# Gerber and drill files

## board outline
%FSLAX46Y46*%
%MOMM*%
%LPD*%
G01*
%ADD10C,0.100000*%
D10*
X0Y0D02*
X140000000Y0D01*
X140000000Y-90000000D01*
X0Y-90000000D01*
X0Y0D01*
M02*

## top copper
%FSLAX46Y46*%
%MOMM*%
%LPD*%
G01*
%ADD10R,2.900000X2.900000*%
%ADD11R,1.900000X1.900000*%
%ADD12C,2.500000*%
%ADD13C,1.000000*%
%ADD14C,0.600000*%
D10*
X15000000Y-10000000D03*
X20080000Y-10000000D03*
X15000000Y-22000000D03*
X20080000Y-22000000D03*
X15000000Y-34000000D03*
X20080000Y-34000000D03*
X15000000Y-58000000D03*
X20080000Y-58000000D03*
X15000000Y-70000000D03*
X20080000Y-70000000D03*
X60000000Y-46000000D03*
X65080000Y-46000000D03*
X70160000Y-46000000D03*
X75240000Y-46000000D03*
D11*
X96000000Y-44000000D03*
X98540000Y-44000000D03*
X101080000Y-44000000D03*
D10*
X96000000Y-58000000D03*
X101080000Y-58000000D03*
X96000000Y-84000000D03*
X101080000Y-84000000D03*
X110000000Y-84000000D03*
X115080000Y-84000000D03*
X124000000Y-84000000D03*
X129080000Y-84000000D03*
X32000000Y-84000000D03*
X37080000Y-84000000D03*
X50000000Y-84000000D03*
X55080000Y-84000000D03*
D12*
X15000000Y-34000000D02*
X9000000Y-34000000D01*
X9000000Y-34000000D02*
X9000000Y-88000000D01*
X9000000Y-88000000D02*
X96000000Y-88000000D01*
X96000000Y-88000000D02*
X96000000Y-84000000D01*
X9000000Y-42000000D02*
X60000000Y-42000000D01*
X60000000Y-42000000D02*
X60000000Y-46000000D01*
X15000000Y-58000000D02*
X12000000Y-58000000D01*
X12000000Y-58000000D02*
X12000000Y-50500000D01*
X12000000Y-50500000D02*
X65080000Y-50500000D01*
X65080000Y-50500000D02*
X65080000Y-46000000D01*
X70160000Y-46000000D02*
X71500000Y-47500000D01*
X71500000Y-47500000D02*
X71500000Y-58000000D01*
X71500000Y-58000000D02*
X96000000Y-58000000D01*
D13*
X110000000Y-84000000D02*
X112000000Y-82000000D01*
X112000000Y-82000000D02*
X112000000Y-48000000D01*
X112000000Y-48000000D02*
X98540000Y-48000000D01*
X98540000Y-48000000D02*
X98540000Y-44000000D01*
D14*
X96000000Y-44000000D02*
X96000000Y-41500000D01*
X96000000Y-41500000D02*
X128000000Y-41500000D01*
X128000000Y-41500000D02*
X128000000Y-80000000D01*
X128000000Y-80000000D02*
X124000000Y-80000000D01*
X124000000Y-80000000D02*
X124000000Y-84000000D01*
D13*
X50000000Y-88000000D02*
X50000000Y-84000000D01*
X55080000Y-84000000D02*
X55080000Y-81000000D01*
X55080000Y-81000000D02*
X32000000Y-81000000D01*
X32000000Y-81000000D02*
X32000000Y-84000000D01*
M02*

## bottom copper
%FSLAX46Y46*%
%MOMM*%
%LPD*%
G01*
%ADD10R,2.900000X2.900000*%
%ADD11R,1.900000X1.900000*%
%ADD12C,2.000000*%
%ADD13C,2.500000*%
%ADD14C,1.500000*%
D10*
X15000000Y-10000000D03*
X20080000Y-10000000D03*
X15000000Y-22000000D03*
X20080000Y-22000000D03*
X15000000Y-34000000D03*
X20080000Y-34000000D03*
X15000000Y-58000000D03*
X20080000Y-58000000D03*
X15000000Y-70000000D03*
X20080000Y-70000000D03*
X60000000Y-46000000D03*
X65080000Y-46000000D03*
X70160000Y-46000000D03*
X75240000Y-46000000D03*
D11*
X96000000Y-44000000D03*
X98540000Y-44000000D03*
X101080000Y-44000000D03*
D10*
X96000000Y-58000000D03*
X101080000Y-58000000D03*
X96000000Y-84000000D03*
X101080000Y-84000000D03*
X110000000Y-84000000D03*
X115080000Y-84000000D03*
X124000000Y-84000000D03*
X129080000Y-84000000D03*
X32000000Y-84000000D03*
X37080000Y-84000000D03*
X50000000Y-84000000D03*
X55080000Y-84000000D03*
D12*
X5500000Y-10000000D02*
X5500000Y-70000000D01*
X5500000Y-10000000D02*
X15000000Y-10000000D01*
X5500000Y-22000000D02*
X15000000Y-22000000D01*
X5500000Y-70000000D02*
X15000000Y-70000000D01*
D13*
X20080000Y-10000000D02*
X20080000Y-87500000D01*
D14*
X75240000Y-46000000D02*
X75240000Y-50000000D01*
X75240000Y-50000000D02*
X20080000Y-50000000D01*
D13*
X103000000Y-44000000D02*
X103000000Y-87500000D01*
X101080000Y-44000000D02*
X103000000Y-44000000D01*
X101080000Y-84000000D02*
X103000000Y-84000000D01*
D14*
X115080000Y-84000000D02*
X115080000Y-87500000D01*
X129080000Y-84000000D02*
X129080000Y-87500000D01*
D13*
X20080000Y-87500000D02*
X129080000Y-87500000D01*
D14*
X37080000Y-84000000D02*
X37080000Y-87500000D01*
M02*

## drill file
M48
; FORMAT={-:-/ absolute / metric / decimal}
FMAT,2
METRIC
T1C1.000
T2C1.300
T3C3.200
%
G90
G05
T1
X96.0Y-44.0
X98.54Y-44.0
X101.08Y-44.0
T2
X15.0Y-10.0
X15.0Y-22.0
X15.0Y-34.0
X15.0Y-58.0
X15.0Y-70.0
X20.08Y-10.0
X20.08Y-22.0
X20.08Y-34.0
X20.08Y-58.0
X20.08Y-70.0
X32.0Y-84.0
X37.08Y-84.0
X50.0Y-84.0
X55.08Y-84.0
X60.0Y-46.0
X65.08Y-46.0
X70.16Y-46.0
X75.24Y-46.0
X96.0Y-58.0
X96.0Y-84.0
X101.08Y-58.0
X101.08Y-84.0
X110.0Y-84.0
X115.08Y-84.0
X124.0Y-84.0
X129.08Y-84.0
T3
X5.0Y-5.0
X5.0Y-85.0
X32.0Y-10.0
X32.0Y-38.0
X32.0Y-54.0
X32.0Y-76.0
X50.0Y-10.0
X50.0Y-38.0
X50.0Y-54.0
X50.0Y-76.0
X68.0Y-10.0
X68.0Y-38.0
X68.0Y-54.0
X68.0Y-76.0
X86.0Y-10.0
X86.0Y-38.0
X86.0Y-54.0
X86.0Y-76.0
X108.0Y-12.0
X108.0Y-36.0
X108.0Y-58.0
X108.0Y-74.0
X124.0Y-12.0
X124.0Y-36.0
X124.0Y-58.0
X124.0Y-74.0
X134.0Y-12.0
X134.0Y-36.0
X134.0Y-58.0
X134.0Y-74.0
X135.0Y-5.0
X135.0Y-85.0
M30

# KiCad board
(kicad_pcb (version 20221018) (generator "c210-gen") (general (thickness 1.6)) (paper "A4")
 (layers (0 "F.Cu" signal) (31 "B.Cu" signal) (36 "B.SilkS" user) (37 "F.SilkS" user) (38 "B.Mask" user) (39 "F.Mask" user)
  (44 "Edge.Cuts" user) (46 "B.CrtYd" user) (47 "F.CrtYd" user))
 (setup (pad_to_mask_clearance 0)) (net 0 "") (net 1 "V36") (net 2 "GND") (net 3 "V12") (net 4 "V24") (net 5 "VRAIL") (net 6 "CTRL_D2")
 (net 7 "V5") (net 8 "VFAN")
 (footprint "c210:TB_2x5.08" (layer "F.Cu") (at 15 10)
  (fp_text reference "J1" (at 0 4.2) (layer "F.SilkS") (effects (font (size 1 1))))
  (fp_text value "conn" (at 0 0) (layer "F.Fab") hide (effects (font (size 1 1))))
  (pad "1" thru_hole rect (at 0.0 0) (size 2.9 2.9) (drill 1.3) (layers "*.Cu" "*.Mask") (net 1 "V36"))
  (pad "2" thru_hole rect (at 5.08 0) (size 2.9 2.9) (drill 1.3) (layers "*.Cu" "*.Mask") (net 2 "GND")))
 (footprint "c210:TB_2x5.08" (layer "F.Cu") (at 15 22)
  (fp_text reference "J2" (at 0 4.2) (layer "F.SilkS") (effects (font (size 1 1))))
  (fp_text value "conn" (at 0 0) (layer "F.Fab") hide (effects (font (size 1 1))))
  (pad "1" thru_hole rect (at 0.0 0) (size 2.9 2.9) (drill 1.3) (layers "*.Cu" "*.Mask") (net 1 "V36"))
  (pad "2" thru_hole rect (at 5.08 0) (size 2.9 2.9) (drill 1.3) (layers "*.Cu" "*.Mask") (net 2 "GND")))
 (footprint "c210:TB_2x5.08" (layer "F.Cu") (at 15 34)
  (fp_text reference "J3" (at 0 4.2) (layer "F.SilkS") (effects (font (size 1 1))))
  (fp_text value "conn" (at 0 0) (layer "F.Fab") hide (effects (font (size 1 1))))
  (pad "1" thru_hole rect (at 0.0 0) (size 2.9 2.9) (drill 1.3) (layers "*.Cu" "*.Mask") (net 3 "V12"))
  (pad "2" thru_hole rect (at 5.08 0) (size 2.9 2.9) (drill 1.3) (layers "*.Cu" "*.Mask") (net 2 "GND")))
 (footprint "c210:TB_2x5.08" (layer "F.Cu") (at 15 58)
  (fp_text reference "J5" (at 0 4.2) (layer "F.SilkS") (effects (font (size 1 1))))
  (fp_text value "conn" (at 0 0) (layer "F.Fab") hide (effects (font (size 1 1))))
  (pad "1" thru_hole rect (at 0.0 0) (size 2.9 2.9) (drill 1.3) (layers "*.Cu" "*.Mask") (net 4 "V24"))
  (pad "2" thru_hole rect (at 5.08 0) (size 2.9 2.9) (drill 1.3) (layers "*.Cu" "*.Mask") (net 2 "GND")))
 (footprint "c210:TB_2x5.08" (layer "F.Cu") (at 15 70)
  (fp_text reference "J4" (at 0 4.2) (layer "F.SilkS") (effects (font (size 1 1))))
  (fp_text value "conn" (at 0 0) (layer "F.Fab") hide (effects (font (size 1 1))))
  (pad "1" thru_hole rect (at 0.0 0) (size 2.9 2.9) (drill 1.3) (layers "*.Cu" "*.Mask") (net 1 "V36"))
  (pad "2" thru_hole rect (at 5.08 0) (size 2.9 2.9) (drill 1.3) (layers "*.Cu" "*.Mask") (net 2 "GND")))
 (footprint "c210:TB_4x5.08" (layer "F.Cu") (at 60 46)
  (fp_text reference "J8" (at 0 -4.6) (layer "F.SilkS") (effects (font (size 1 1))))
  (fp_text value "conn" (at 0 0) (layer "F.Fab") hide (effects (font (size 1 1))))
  (pad "1" thru_hole rect (at 0.0 0) (size 2.9 2.9) (drill 1.3) (layers "*.Cu" "*.Mask") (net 3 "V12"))
  (pad "2" thru_hole rect (at 5.08 0) (size 2.9 2.9) (drill 1.3) (layers "*.Cu" "*.Mask") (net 4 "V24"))
  (pad "3" thru_hole rect (at 10.16 0) (size 2.9 2.9) (drill 1.3) (layers "*.Cu" "*.Mask") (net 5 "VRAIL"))
  (pad "4" thru_hole rect (at 15.24 0) (size 2.9 2.9) (drill 1.3) (layers "*.Cu" "*.Mask") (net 2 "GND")))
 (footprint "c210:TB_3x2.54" (layer "F.Cu") (at 96 44)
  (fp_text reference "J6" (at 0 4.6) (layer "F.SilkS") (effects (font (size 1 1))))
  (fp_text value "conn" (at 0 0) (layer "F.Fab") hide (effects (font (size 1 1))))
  (pad "1" thru_hole rect (at 0.0 0) (size 1.9 1.9) (drill 1.0) (layers "*.Cu" "*.Mask") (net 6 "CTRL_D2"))
  (pad "2" thru_hole rect (at 2.54 0) (size 1.9 1.9) (drill 1.0) (layers "*.Cu" "*.Mask") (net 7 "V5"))
  (pad "3" thru_hole rect (at 5.08 0) (size 1.9 1.9) (drill 1.0) (layers "*.Cu" "*.Mask") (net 2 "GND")))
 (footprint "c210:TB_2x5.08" (layer "F.Cu") (at 96 58)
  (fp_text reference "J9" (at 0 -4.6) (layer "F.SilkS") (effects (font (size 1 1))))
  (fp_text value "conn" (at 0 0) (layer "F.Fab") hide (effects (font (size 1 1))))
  (pad "1" thru_hole rect (at 0.0 0) (size 2.9 2.9) (drill 1.3) (layers "*.Cu" "*.Mask") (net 5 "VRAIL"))
  (pad "2" thru_hole rect (at 5.08 0) (size 2.9 2.9) (drill 1.3) (layers "*.Cu" "*.Mask") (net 2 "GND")))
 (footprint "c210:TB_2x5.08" (layer "F.Cu") (at 96 84)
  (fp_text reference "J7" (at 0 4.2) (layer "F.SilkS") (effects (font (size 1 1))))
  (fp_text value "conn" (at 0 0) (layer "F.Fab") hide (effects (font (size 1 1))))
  (pad "1" thru_hole rect (at 0.0 0) (size 2.9 2.9) (drill 1.3) (layers "*.Cu" "*.Mask") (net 3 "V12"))
  (pad "2" thru_hole rect (at 5.08 0) (size 2.9 2.9) (drill 1.3) (layers "*.Cu" "*.Mask") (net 2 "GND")))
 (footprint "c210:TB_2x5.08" (layer "F.Cu") (at 110 84)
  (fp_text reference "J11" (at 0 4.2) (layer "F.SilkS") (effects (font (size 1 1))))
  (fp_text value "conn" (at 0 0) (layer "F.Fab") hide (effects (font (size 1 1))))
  (pad "1" thru_hole rect (at 0.0 0) (size 2.9 2.9) (drill 1.3) (layers "*.Cu" "*.Mask") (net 7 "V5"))
  (pad "2" thru_hole rect (at 5.08 0) (size 2.9 2.9) (drill 1.3) (layers "*.Cu" "*.Mask") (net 2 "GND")))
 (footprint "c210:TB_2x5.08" (layer "F.Cu") (at 124 84)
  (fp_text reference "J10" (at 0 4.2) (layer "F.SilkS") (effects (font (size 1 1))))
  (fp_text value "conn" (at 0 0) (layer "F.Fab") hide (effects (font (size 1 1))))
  (pad "1" thru_hole rect (at 0.0 0) (size 2.9 2.9) (drill 1.3) (layers "*.Cu" "*.Mask") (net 6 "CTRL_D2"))
  (pad "2" thru_hole rect (at 5.08 0) (size 2.9 2.9) (drill 1.3) (layers "*.Cu" "*.Mask") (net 2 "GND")))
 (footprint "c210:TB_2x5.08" (layer "F.Cu") (at 32 84)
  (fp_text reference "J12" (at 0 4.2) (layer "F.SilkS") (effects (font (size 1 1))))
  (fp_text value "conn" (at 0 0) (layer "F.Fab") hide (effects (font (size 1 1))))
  (pad "1" thru_hole rect (at 0.0 0) (size 2.9 2.9) (drill 1.3) (layers "*.Cu" "*.Mask") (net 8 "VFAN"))
  (pad "2" thru_hole rect (at 5.08 0) (size 2.9 2.9) (drill 1.3) (layers "*.Cu" "*.Mask") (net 2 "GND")))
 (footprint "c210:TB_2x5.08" (layer "F.Cu") (at 50 84)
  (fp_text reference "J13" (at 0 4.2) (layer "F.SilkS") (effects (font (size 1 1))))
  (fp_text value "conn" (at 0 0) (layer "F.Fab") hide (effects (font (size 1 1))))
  (pad "1" thru_hole rect (at 0.0 0) (size 2.9 2.9) (drill 1.3) (layers "*.Cu" "*.Mask") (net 3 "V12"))
  (pad "2" thru_hole rect (at 5.08 0) (size 2.9 2.9) (drill 1.3) (layers "*.Cu" "*.Mask") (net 8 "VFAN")))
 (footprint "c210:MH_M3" (layer "F.Cu") (at 5 5)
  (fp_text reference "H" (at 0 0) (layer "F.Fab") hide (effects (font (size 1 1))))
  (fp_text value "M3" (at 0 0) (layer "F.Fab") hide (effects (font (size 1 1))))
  (pad "" np_thru_hole circle (at 0 0) (size 3.2 3.2) (drill 3.2) (layers "F.Mask" "B.Mask")))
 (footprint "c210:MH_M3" (layer "F.Cu") (at 135 5)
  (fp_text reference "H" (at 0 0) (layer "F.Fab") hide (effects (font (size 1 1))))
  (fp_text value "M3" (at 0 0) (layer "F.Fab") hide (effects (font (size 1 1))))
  (pad "" np_thru_hole circle (at 0 0) (size 3.2 3.2) (drill 3.2) (layers "F.Mask" "B.Mask")))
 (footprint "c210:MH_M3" (layer "F.Cu") (at 5 85)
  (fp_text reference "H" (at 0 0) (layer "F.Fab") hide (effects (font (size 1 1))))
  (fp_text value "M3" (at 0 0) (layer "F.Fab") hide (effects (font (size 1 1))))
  (pad "" np_thru_hole circle (at 0 0) (size 3.2 3.2) (drill 3.2) (layers "F.Mask" "B.Mask")))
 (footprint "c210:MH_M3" (layer "F.Cu") (at 135 85)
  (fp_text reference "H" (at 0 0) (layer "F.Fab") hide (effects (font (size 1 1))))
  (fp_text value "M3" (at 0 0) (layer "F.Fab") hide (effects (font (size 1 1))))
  (pad "" np_thru_hole circle (at 0 0) (size 3.2 3.2) (drill 3.2) (layers "F.Mask" "B.Mask")))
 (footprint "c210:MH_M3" (layer "F.Cu") (at 32 10)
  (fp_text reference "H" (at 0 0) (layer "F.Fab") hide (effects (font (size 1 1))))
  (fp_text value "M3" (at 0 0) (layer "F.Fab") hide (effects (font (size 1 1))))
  (pad "" np_thru_hole circle (at 0 0) (size 3.2 3.2) (drill 3.2) (layers "F.Mask" "B.Mask")))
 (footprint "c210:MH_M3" (layer "F.Cu") (at 32 38)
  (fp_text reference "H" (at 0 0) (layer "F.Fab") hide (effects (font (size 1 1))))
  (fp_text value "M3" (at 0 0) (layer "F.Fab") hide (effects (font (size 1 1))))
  (pad "" np_thru_hole circle (at 0 0) (size 3.2 3.2) (drill 3.2) (layers "F.Mask" "B.Mask")))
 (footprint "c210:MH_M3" (layer "F.Cu") (at 32 54)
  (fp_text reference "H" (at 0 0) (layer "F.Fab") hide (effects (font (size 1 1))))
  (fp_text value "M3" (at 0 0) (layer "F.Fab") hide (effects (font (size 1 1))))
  (pad "" np_thru_hole circle (at 0 0) (size 3.2 3.2) (drill 3.2) (layers "F.Mask" "B.Mask")))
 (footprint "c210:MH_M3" (layer "F.Cu") (at 32 76)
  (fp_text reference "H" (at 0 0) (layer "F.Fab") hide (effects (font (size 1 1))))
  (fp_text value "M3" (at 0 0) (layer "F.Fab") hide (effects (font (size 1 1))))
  (pad "" np_thru_hole circle (at 0 0) (size 3.2 3.2) (drill 3.2) (layers "F.Mask" "B.Mask")))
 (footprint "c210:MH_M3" (layer "F.Cu") (at 50 10)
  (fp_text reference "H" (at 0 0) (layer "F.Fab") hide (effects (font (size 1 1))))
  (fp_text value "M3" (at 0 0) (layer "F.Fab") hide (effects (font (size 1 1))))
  (pad "" np_thru_hole circle (at 0 0) (size 3.2 3.2) (drill 3.2) (layers "F.Mask" "B.Mask")))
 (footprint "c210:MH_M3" (layer "F.Cu") (at 50 38)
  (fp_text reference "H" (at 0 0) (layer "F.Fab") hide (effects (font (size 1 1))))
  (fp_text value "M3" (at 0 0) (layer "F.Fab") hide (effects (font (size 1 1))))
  (pad "" np_thru_hole circle (at 0 0) (size 3.2 3.2) (drill 3.2) (layers "F.Mask" "B.Mask")))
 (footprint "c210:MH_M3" (layer "F.Cu") (at 50 54)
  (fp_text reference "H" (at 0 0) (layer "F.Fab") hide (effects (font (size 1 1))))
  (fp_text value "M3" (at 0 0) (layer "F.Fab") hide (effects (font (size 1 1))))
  (pad "" np_thru_hole circle (at 0 0) (size 3.2 3.2) (drill 3.2) (layers "F.Mask" "B.Mask")))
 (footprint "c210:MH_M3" (layer "F.Cu") (at 50 76)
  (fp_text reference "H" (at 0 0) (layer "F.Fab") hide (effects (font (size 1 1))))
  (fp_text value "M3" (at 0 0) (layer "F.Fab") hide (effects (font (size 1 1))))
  (pad "" np_thru_hole circle (at 0 0) (size 3.2 3.2) (drill 3.2) (layers "F.Mask" "B.Mask")))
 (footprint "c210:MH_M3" (layer "F.Cu") (at 68 10)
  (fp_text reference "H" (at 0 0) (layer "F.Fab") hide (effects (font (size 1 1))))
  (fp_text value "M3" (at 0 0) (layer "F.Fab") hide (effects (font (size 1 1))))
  (pad "" np_thru_hole circle (at 0 0) (size 3.2 3.2) (drill 3.2) (layers "F.Mask" "B.Mask")))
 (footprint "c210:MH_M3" (layer "F.Cu") (at 68 38)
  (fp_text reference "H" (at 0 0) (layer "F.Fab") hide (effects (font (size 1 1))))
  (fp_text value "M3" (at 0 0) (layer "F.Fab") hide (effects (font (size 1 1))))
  (pad "" np_thru_hole circle (at 0 0) (size 3.2 3.2) (drill 3.2) (layers "F.Mask" "B.Mask")))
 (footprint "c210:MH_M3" (layer "F.Cu") (at 68 54)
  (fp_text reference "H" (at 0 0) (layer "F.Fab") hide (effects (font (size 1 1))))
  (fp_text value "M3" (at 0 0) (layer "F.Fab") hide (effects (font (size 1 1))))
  (pad "" np_thru_hole circle (at 0 0) (size 3.2 3.2) (drill 3.2) (layers "F.Mask" "B.Mask")))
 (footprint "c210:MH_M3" (layer "F.Cu") (at 68 76)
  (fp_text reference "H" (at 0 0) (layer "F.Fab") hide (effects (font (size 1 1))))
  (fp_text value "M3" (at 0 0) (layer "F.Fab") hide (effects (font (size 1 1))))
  (pad "" np_thru_hole circle (at 0 0) (size 3.2 3.2) (drill 3.2) (layers "F.Mask" "B.Mask")))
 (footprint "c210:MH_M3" (layer "F.Cu") (at 86 10)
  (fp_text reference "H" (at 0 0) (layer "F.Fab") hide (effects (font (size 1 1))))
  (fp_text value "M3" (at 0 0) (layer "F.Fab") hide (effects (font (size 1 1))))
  (pad "" np_thru_hole circle (at 0 0) (size 3.2 3.2) (drill 3.2) (layers "F.Mask" "B.Mask")))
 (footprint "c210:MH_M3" (layer "F.Cu") (at 86 38)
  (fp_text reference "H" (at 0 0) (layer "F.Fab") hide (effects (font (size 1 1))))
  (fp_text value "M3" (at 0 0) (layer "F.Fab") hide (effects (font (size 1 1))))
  (pad "" np_thru_hole circle (at 0 0) (size 3.2 3.2) (drill 3.2) (layers "F.Mask" "B.Mask")))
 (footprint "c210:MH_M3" (layer "F.Cu") (at 86 54)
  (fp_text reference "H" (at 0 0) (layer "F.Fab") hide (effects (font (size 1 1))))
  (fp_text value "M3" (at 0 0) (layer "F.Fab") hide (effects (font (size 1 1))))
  (pad "" np_thru_hole circle (at 0 0) (size 3.2 3.2) (drill 3.2) (layers "F.Mask" "B.Mask")))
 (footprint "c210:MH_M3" (layer "F.Cu") (at 86 76)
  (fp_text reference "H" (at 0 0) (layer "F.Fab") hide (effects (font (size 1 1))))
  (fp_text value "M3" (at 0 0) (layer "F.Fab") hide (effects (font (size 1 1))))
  (pad "" np_thru_hole circle (at 0 0) (size 3.2 3.2) (drill 3.2) (layers "F.Mask" "B.Mask")))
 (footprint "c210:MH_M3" (layer "F.Cu") (at 108 12)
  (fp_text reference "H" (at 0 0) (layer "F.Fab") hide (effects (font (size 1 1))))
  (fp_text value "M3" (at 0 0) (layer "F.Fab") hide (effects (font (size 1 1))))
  (pad "" np_thru_hole circle (at 0 0) (size 3.2 3.2) (drill 3.2) (layers "F.Mask" "B.Mask")))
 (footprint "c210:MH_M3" (layer "F.Cu") (at 108 36)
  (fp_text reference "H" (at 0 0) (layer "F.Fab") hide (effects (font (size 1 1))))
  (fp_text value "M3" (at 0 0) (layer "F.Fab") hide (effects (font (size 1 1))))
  (pad "" np_thru_hole circle (at 0 0) (size 3.2 3.2) (drill 3.2) (layers "F.Mask" "B.Mask")))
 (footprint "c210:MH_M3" (layer "F.Cu") (at 108 58)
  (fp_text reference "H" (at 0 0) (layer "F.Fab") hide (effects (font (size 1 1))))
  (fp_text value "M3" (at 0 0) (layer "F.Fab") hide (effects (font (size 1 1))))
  (pad "" np_thru_hole circle (at 0 0) (size 3.2 3.2) (drill 3.2) (layers "F.Mask" "B.Mask")))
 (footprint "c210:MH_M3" (layer "F.Cu") (at 108 74)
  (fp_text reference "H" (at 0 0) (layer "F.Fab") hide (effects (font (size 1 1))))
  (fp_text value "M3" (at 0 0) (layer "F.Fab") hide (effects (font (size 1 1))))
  (pad "" np_thru_hole circle (at 0 0) (size 3.2 3.2) (drill 3.2) (layers "F.Mask" "B.Mask")))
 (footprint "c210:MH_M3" (layer "F.Cu") (at 124 12)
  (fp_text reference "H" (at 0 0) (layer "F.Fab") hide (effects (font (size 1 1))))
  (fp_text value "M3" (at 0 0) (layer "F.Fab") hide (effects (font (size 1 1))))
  (pad "" np_thru_hole circle (at 0 0) (size 3.2 3.2) (drill 3.2) (layers "F.Mask" "B.Mask")))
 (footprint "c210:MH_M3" (layer "F.Cu") (at 124 36)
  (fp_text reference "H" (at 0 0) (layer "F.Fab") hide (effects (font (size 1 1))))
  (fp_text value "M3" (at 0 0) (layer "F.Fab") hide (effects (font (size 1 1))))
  (pad "" np_thru_hole circle (at 0 0) (size 3.2 3.2) (drill 3.2) (layers "F.Mask" "B.Mask")))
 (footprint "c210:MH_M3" (layer "F.Cu") (at 124 58)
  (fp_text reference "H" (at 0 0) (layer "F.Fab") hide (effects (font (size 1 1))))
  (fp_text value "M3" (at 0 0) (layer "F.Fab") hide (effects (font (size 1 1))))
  (pad "" np_thru_hole circle (at 0 0) (size 3.2 3.2) (drill 3.2) (layers "F.Mask" "B.Mask")))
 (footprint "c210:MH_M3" (layer "F.Cu") (at 124 74)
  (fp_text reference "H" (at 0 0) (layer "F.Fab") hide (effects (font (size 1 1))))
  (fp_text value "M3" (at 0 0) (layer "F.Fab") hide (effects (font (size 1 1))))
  (pad "" np_thru_hole circle (at 0 0) (size 3.2 3.2) (drill 3.2) (layers "F.Mask" "B.Mask")))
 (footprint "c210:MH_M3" (layer "F.Cu") (at 134 12)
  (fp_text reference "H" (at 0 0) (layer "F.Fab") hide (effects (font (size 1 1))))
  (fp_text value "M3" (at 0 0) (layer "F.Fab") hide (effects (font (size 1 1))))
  (pad "" np_thru_hole circle (at 0 0) (size 3.2 3.2) (drill 3.2) (layers "F.Mask" "B.Mask")))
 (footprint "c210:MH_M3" (layer "F.Cu") (at 134 36)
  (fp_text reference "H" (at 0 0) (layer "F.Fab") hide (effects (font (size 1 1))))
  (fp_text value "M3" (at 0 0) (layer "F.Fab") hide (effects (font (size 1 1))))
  (pad "" np_thru_hole circle (at 0 0) (size 3.2 3.2) (drill 3.2) (layers "F.Mask" "B.Mask")))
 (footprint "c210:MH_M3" (layer "F.Cu") (at 134 58)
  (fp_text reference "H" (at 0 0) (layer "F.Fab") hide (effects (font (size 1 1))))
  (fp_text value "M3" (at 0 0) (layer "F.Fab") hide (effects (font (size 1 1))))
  (pad "" np_thru_hole circle (at 0 0) (size 3.2 3.2) (drill 3.2) (layers "F.Mask" "B.Mask")))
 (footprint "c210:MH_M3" (layer "F.Cu") (at 134 74)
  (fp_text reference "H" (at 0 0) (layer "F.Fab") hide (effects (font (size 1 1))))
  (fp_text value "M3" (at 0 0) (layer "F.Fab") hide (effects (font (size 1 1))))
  (pad "" np_thru_hole circle (at 0 0) (size 3.2 3.2) (drill 3.2) (layers "F.Mask" "B.Mask")))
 (segment (start 5.5 10) (end 5.5 70) (width 2.0) (layer "B.Cu") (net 1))
 (segment (start 5.5 10) (end 15.0 10) (width 2.0) (layer "B.Cu") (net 1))
 (segment (start 5.5 22) (end 15.0 22) (width 2.0) (layer "B.Cu") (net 1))
 (segment (start 5.5 70) (end 15.0 70) (width 2.0) (layer "B.Cu") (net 1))
 (segment (start 20.08 10) (end 20.08 87.5) (width 2.5) (layer "B.Cu") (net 2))
 (segment (start 75.24 46) (end 75.24 50) (width 1.5) (layer "B.Cu") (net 2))
 (segment (start 75.24 50) (end 20.08 50) (width 1.5) (layer "B.Cu") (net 2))
 (segment (start 103 44) (end 103 87.5) (width 2.5) (layer "B.Cu") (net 2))
 (segment (start 101.08 44) (end 103 44) (width 2.5) (layer "B.Cu") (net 2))
 (segment (start 101.08 84) (end 103 84) (width 2.5) (layer "B.Cu") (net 2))
 (segment (start 115.08 84) (end 115.08 87.5) (width 1.5) (layer "B.Cu") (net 2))
 (segment (start 129.08 84) (end 129.08 87.5) (width 1.5) (layer "B.Cu") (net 2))
 (segment (start 20.08 87.5) (end 129.08 87.5) (width 2.5) (layer "B.Cu") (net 2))
 (segment (start 15.0 34) (end 9 34) (width 2.5) (layer "F.Cu") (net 3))
 (segment (start 9 34) (end 9 88) (width 2.5) (layer "F.Cu") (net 3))
 (segment (start 9 88) (end 96 88) (width 2.5) (layer "F.Cu") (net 3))
 (segment (start 96 88) (end 96.0 84) (width 2.5) (layer "F.Cu") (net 3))
 (segment (start 9 42) (end 60 42) (width 2.5) (layer "F.Cu") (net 3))
 (segment (start 60 42) (end 60.0 46) (width 2.5) (layer "F.Cu") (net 3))
 (segment (start 15.0 58) (end 12 58) (width 2.5) (layer "F.Cu") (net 4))
 (segment (start 12 58) (end 12 50.5) (width 2.5) (layer "F.Cu") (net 4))
 (segment (start 12 50.5) (end 65.08 50.5) (width 2.5) (layer "F.Cu") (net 4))
 (segment (start 65.08 50.5) (end 65.08 46) (width 2.5) (layer "F.Cu") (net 4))
 (segment (start 70.16 46) (end 71.5 47.5) (width 2.5) (layer "F.Cu") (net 5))
 (segment (start 71.5 47.5) (end 71.5 58) (width 2.5) (layer "F.Cu") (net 5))
 (segment (start 71.5 58) (end 96.0 58) (width 2.5) (layer "F.Cu") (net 5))
 (segment (start 110.0 84) (end 112 82) (width 1.0) (layer "F.Cu") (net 7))
 (segment (start 112 82) (end 112 48) (width 1.0) (layer "F.Cu") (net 7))
 (segment (start 112 48) (end 98.54 48) (width 1.0) (layer "F.Cu") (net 7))
 (segment (start 98.54 48) (end 98.54 44) (width 1.0) (layer "F.Cu") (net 7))
 (segment (start 96.0 44) (end 96 41.5) (width 0.6) (layer "F.Cu") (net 6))
 (segment (start 96 41.5) (end 128 41.5) (width 0.6) (layer "F.Cu") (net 6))
 (segment (start 128 41.5) (end 128 80) (width 0.6) (layer "F.Cu") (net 6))
 (segment (start 128 80) (end 124 80) (width 0.6) (layer "F.Cu") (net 6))
 (segment (start 124 80) (end 124.0 84) (width 0.6) (layer "F.Cu") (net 6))
 (segment (start 50 88) (end 50.0 84) (width 1.0) (layer "F.Cu") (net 3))
 (segment (start 55.08 84) (end 55.08 81) (width 1.0) (layer "F.Cu") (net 8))
 (segment (start 55.08 81) (end 32 81) (width 1.0) (layer "F.Cu") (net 8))
 (segment (start 32 81) (end 32.0 84) (width 1.0) (layer "F.Cu") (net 8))
 (segment (start 37.08 84) (end 37.08 87.5) (width 1.5) (layer "B.Cu") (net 2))
 (gr_rect (start 0 0) (end 140 90) (stroke (width 0.1) (type default)) (fill none) (layer "Edge.Cuts")))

